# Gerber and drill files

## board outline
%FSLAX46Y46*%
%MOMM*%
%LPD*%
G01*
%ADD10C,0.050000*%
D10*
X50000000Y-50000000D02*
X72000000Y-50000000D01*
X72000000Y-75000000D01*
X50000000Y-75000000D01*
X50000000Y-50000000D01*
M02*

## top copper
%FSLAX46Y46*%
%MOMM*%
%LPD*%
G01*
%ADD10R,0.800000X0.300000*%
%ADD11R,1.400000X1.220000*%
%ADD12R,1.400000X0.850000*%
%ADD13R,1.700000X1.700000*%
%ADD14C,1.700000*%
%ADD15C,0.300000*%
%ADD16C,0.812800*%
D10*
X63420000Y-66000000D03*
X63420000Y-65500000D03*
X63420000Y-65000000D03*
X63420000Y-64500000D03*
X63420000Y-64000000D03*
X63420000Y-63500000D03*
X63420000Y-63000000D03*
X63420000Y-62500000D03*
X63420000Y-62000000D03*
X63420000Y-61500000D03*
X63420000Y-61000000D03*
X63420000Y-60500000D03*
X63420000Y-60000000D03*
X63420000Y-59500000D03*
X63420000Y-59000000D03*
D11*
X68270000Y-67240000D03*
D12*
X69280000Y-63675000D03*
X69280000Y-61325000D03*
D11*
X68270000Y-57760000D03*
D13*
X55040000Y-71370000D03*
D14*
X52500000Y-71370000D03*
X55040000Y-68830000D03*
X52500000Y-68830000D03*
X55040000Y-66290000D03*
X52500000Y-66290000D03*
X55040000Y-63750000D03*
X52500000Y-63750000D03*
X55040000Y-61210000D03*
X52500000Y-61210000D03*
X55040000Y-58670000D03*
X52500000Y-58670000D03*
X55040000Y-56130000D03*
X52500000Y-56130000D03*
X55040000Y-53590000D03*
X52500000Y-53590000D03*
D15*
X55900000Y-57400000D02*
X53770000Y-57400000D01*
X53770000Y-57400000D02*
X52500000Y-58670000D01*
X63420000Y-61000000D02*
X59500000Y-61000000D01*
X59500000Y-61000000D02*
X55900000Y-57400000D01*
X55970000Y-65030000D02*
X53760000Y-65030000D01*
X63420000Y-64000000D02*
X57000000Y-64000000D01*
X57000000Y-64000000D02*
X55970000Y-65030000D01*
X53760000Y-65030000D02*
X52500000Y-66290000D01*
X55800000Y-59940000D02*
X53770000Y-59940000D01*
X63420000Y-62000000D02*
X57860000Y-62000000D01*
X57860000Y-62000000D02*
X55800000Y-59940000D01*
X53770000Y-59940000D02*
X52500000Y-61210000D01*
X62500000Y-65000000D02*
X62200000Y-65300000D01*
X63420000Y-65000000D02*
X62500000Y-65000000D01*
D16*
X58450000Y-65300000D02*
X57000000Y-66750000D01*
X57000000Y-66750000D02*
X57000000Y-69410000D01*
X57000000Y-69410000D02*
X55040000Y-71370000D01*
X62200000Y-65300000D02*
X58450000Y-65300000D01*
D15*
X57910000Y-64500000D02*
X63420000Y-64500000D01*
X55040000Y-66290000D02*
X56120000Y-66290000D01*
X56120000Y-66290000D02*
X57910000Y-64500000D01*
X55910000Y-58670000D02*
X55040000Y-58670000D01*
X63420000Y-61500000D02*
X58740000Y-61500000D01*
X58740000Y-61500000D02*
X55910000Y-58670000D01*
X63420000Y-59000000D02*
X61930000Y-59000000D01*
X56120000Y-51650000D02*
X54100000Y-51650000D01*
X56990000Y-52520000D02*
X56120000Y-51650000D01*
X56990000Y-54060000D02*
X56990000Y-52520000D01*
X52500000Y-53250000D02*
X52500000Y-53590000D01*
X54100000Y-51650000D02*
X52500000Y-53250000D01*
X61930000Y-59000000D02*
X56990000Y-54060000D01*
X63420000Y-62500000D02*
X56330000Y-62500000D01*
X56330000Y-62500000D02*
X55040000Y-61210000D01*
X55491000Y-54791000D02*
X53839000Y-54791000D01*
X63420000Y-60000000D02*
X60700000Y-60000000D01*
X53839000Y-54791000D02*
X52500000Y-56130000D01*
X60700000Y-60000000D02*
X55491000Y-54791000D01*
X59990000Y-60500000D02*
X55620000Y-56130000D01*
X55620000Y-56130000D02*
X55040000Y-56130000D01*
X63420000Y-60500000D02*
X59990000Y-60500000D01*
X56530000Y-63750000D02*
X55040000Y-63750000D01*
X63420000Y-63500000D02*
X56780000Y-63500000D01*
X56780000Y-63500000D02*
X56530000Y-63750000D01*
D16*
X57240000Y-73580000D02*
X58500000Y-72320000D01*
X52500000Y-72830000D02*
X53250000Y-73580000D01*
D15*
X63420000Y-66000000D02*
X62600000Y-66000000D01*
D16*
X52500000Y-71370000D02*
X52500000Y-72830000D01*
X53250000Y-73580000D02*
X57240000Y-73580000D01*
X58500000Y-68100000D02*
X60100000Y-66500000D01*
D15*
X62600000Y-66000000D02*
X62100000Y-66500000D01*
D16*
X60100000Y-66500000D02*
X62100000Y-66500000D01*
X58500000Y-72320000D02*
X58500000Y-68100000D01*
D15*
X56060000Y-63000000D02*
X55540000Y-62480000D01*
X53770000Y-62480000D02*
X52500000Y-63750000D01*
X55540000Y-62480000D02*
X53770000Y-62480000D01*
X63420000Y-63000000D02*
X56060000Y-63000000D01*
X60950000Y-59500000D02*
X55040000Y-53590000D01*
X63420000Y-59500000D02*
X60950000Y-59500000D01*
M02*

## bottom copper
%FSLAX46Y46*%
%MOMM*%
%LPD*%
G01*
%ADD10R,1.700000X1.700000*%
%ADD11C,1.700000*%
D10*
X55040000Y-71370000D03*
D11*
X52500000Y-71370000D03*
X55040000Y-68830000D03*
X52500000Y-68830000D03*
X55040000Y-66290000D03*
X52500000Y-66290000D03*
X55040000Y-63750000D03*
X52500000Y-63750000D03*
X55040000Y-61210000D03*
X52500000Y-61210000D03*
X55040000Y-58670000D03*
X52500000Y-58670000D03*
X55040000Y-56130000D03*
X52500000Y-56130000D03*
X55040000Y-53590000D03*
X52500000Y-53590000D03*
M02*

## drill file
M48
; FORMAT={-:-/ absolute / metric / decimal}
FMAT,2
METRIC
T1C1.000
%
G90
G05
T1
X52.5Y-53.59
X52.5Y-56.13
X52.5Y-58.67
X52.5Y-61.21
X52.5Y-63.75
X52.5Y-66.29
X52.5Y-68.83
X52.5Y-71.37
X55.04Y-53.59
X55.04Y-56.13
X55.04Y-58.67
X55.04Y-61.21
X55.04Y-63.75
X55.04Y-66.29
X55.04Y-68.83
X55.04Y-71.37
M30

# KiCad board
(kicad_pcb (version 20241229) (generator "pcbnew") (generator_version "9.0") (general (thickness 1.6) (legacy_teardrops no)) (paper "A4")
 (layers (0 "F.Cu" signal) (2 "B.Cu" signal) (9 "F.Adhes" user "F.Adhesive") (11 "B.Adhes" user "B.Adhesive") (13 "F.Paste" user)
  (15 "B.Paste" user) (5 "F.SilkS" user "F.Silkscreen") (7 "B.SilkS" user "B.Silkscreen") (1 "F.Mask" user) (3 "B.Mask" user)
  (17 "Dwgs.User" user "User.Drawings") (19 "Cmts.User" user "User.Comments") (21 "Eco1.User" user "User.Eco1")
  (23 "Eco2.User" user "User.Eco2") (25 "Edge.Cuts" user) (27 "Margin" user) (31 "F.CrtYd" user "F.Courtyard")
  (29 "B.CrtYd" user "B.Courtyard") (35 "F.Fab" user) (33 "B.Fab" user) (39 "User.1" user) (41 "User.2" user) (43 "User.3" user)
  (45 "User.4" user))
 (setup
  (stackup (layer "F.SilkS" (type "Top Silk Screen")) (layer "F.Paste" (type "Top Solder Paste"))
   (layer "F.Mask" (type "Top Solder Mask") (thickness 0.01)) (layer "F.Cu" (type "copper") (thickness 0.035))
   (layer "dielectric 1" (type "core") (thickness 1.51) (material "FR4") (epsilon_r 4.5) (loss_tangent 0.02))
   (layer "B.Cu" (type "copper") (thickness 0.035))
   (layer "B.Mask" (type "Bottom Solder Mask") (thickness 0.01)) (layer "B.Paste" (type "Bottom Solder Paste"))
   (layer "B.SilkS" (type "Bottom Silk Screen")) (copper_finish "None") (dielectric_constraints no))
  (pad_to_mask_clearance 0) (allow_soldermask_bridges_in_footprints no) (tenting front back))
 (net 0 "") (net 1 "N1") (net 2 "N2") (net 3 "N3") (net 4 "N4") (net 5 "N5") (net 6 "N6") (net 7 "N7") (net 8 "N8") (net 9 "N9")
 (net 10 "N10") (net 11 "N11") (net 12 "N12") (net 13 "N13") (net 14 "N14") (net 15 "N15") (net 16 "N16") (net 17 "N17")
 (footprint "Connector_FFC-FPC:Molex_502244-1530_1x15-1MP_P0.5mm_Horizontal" (layer "F.Cu") (at 66.5 62.5 90)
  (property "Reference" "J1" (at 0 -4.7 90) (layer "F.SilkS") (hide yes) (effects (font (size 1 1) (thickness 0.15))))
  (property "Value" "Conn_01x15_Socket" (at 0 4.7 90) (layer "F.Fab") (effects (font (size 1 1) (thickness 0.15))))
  (pad "1" smd rect (at -3.5 -3.08 90) (size 0.3 0.8) (layers "F.Cu" "F.Mask" "F.Paste") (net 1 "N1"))
  (pad "2" smd rect (at -3 -3.08 90) (size 0.3 0.8) (layers "F.Cu" "F.Mask" "F.Paste") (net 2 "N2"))
  (pad "3" smd rect (at -2.5 -3.08 90) (size 0.3 0.8) (layers "F.Cu" "F.Mask" "F.Paste") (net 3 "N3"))
  (pad "4" smd rect (at -2 -3.08 90) (size 0.3 0.8) (layers "F.Cu" "F.Mask" "F.Paste") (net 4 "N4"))
  (pad "5" smd rect (at -1.5 -3.08 90) (size 0.3 0.8) (layers "F.Cu" "F.Mask" "F.Paste") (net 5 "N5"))
  (pad "6" smd rect (at -1 -3.08 90) (size 0.3 0.8) (layers "F.Cu" "F.Mask" "F.Paste") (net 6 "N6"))
  (pad "7" smd rect (at -0.5 -3.08 90) (size 0.3 0.8) (layers "F.Cu" "F.Mask" "F.Paste") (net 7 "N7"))
  (pad "8" smd rect (at 0 -3.08 90) (size 0.3 0.8) (layers "F.Cu" "F.Mask" "F.Paste") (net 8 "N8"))
  (pad "9" smd rect (at 0.5 -3.08 90) (size 0.3 0.8) (layers "F.Cu" "F.Mask" "F.Paste") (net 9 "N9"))
  (pad "10" smd rect (at 1 -3.08 90) (size 0.3 0.8) (layers "F.Cu" "F.Mask" "F.Paste") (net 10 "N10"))
  (pad "11" smd rect (at 1.5 -3.08 90) (size 0.3 0.8) (layers "F.Cu" "F.Mask" "F.Paste") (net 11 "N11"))
  (pad "12" smd rect (at 2 -3.08 90) (size 0.3 0.8) (layers "F.Cu" "F.Mask" "F.Paste") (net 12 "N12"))
  (pad "13" smd rect (at 2.5 -3.08 90) (size 0.3 0.8) (layers "F.Cu" "F.Mask" "F.Paste") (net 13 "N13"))
  (pad "14" smd rect (at 3 -3.08 90) (size 0.3 0.8) (layers "F.Cu" "F.Mask" "F.Paste") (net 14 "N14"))
  (pad "15" smd rect (at 3.5 -3.08 90) (size 0.3 0.8) (layers "F.Cu" "F.Mask" "F.Paste") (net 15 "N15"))
  (pad "MP" smd rect (at -4.74 1.77 90) (size 1.22 1.4) (layers "F.Cu" "F.Mask" "F.Paste"))
  (pad "MP" smd rect (at -1.175 2.78 90) (size 0.85 1.4) (layers "F.Cu" "F.Mask" "F.Paste"))
  (pad "MP" smd rect (at 1.175 2.78 90) (size 0.85 1.4) (layers "F.Cu" "F.Mask" "F.Paste"))
  (pad "MP" smd rect (at 4.74 1.77 90) (size 1.22 1.4) (layers "F.Cu" "F.Mask" "F.Paste"))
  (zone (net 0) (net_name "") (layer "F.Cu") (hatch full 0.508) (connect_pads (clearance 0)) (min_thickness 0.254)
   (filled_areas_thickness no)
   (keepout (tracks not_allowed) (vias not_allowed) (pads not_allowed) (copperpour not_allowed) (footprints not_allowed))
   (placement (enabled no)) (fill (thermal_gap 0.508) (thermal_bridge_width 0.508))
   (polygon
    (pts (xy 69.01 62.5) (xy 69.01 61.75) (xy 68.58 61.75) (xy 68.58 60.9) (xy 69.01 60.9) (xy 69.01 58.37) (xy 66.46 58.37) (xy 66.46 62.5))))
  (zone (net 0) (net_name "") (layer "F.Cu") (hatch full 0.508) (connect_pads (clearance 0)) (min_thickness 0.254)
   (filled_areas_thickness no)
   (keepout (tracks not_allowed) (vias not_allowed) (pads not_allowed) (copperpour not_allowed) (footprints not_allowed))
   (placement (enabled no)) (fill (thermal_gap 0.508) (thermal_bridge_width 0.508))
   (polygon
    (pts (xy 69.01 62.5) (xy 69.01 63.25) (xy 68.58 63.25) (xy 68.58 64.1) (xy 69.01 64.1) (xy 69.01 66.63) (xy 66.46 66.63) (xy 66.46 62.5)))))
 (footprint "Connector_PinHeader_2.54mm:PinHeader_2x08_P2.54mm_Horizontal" (layer "F.Cu") (at 55.04 71.37 180)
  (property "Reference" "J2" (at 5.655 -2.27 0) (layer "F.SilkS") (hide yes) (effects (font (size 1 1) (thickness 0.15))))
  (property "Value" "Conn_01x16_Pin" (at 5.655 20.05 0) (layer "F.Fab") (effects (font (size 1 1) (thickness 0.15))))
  (pad "1" thru_hole rect (at 0 0 180) (size 1.7 1.7) (drill 1) (layers "*.Cu" "*.Mask") (remove_unused_layers no) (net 3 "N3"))
  (pad "2" thru_hole circle (at 2.54 0 180) (size 1.7 1.7) (drill 1) (layers "*.Cu" "*.Mask") (remove_unused_layers no) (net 1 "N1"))
  (pad "3" thru_hole circle (at 0 2.54 180) (size 1.7 1.7) (drill 1) (layers "*.Cu" "*.Mask") (remove_unused_layers no) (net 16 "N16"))
  (pad "4" thru_hole circle (at 2.54 2.54 180) (size 1.7 1.7) (drill 1) (layers "*.Cu" "*.Mask") (remove_unused_layers no) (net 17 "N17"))
  (pad "5" thru_hole circle (at 0 5.08 180) (size 1.7 1.7) (drill 1) (layers "*.Cu" "*.Mask") (remove_unused_layers no) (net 4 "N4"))
  (pad "6" thru_hole circle (at 2.54 5.08 180) (size 1.7 1.7) (drill 1) (layers "*.Cu" "*.Mask") (remove_unused_layers no) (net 5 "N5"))
  (pad "7" thru_hole circle (at 0 7.62 180) (size 1.7 1.7) (drill 1) (layers "*.Cu" "*.Mask") (remove_unused_layers no) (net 6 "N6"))
  (pad "8" thru_hole circle (at 2.54 7.62 180) (size 1.7 1.7) (drill 1) (layers "*.Cu" "*.Mask") (remove_unused_layers no) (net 7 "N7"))
  (pad "9" thru_hole circle (at 0 10.16 180) (size 1.7 1.7) (drill 1) (layers "*.Cu" "*.Mask") (remove_unused_layers no) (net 8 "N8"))
  (pad "10" thru_hole circle (at 2.54 10.16 180) (size 1.7 1.7) (drill 1) (layers "*.Cu" "*.Mask") (remove_unused_layers no) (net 9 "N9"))
  (pad "11" thru_hole circle (at 0 12.7 180) (size 1.7 1.7) (drill 1) (layers "*.Cu" "*.Mask") (remove_unused_layers no) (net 10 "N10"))
  (pad "12" thru_hole circle (at 2.54 12.7 180) (size 1.7 1.7) (drill 1) (layers "*.Cu" "*.Mask") (remove_unused_layers no) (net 11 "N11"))
  (pad "13" thru_hole circle (at 0 15.24 180) (size 1.7 1.7) (drill 1) (layers "*.Cu" "*.Mask") (remove_unused_layers no) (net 12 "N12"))
  (pad "14" thru_hole circle (at 2.54 15.24 180) (size 1.7 1.7) (drill 1) (layers "*.Cu" "*.Mask") (remove_unused_layers no) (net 13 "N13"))
  (pad "15" thru_hole circle (at 0 17.78 180) (size 1.7 1.7) (drill 1) (layers "*.Cu" "*.Mask") (remove_unused_layers no) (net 14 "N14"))
  (pad "16" thru_hole circle (at 2.54 17.78 180) (size 1.7 1.7) (drill 1) (layers "*.Cu" "*.Mask") (remove_unused_layers no) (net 15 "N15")))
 (gr_rect (start 50 50) (end 72 75) (stroke (width 0.05) (type solid)) (fill no) (layer "Edge.Cuts"))
 (segment (start 55.9 57.4) (end 53.77 57.4) (width 0.3) (layer "F.Cu") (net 11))
 (segment (start 53.77 57.4) (end 52.5 58.67) (width 0.3) (layer "F.Cu") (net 11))
 (segment (start 63.42 61) (end 59.5 61) (width 0.3) (layer "F.Cu") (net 11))
 (segment (start 59.5 61) (end 55.9 57.4) (width 0.3) (layer "F.Cu") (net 11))
 (segment (start 55.97 65.03) (end 53.76 65.03) (width 0.3) (layer "F.Cu") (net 5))
 (segment (start 63.42 64) (end 57 64) (width 0.3) (layer "F.Cu") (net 5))
 (segment (start 57 64) (end 55.97 65.03) (width 0.3) (layer "F.Cu") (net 5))
 (segment (start 53.76 65.03) (end 52.5 66.29) (width 0.3) (layer "F.Cu") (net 5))
 (segment (start 55.8 59.94) (end 53.77 59.94) (width 0.3) (layer "F.Cu") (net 9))
 (segment (start 63.42 62) (end 57.86 62) (width 0.3) (layer "F.Cu") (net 9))
 (segment (start 57.86 62) (end 55.8 59.94) (width 0.3) (layer "F.Cu") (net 9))
 (segment (start 53.77 59.94) (end 52.5 61.21) (width 0.3) (layer "F.Cu") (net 9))
 (segment (start 62.5 65) (end 62.2 65.3) (width 0.3) (layer "F.Cu") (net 3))
 (segment (start 63.42 65) (end 62.5 65) (width 0.3) (layer "F.Cu") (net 3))
 (segment (start 58.45 65.3) (end 57 66.75) (width 0.8128) (layer "F.Cu") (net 3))
 (segment (start 57 66.75) (end 57 69.41) (width 0.8128) (layer "F.Cu") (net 3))
 (segment (start 57 69.41) (end 55.04 71.37) (width 0.8128) (layer "F.Cu") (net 3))
 (segment (start 62.2 65.3) (end 58.45 65.3) (width 0.8128) (layer "F.Cu") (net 3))
 (segment (start 57.91 64.5) (end 63.42 64.5) (width 0.3) (layer "F.Cu") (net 4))
 (segment (start 55.04 66.29) (end 56.12 66.29) (width 0.3) (layer "F.Cu") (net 4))
 (segment (start 56.12 66.29) (end 57.91 64.5) (width 0.3) (layer "F.Cu") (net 4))
 (segment (start 55.91 58.67) (end 55.04 58.67) (width 0.3) (layer "F.Cu") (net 10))
 (segment (start 63.42 61.5) (end 58.74 61.5) (width 0.3) (layer "F.Cu") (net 10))
 (segment (start 58.74 61.5) (end 55.91 58.67) (width 0.3) (layer "F.Cu") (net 10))
 (segment (start 63.42 59) (end 61.93 59) (width 0.3) (layer "F.Cu") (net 15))
 (segment (start 56.12 51.65) (end 54.1 51.65) (width 0.3) (layer "F.Cu") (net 15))
 (segment (start 56.99 52.52) (end 56.12 51.65) (width 0.3) (layer "F.Cu") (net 15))
 (segment (start 56.99 54.06) (end 56.99 52.52) (width 0.3) (layer "F.Cu") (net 15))
 (segment (start 52.5 53.25) (end 52.5 53.59) (width 0.3) (layer "F.Cu") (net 15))
 (segment (start 54.1 51.65) (end 52.5 53.25) (width 0.3) (layer "F.Cu") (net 15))
 (segment (start 61.93 59) (end 56.99 54.06) (width 0.3) (layer "F.Cu") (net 15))
 (segment (start 63.42 62.5) (end 56.33 62.5) (width 0.3) (layer "F.Cu") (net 8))
 (segment (start 56.33 62.5) (end 55.04 61.21) (width 0.3) (layer "F.Cu") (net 8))
 (segment (start 55.491 54.791) (end 53.839 54.791) (width 0.3) (layer "F.Cu") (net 13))
 (segment (start 63.42 60) (end 60.7 60) (width 0.3) (layer "F.Cu") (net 13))
 (segment (start 53.839 54.791) (end 52.5 56.13) (width 0.3) (layer "F.Cu") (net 13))
 (segment (start 60.7 60) (end 55.491 54.791) (width 0.3) (layer "F.Cu") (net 13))
 (segment (start 59.99 60.5) (end 55.62 56.13) (width 0.3) (layer "F.Cu") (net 12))
 (segment (start 55.62 56.13) (end 55.04 56.13) (width 0.3) (layer "F.Cu") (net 12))
 (segment (start 63.42 60.5) (end 59.99 60.5) (width 0.3) (layer "F.Cu") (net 12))
 (segment (start 56.53 63.75) (end 55.04 63.75) (width 0.3) (layer "F.Cu") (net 6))
 (segment (start 63.42 63.5) (end 56.78 63.5) (width 0.3) (layer "F.Cu") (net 6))
 (segment (start 56.78 63.5) (end 56.53 63.75) (width 0.3) (layer "F.Cu") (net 6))
 (segment (start 57.24 73.58) (end 58.5 72.32) (width 0.8128) (layer "F.Cu") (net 1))
 (segment (start 52.5 72.83) (end 53.25 73.58) (width 0.8128) (layer "F.Cu") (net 1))
 (segment (start 63.42 66) (end 62.6 66) (width 0.3) (layer "F.Cu") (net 1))
 (segment (start 52.5 71.37) (end 52.5 72.83) (width 0.8128) (layer "F.Cu") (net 1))
 (segment (start 53.25 73.58) (end 57.24 73.58) (width 0.8128) (layer "F.Cu") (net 1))
 (segment (start 58.5 68.1) (end 60.1 66.5) (width 0.8128) (layer "F.Cu") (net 1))
 (segment (start 62.6 66) (end 62.1 66.5) (width 0.3) (layer "F.Cu") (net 1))
 (segment (start 60.1 66.5) (end 62.1 66.5) (width 0.8128) (layer "F.Cu") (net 1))
 (segment (start 58.5 72.32) (end 58.5 68.1) (width 0.8128) (layer "F.Cu") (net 1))
 (segment (start 56.06 63) (end 55.54 62.48) (width 0.3) (layer "F.Cu") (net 7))
 (segment (start 53.77 62.48) (end 52.5 63.75) (width 0.3) (layer "F.Cu") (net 7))
 (segment (start 55.54 62.48) (end 53.77 62.48) (width 0.3) (layer "F.Cu") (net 7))
 (segment (start 63.42 63) (end 56.06 63) (width 0.3) (layer "F.Cu") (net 7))
 (segment (start 60.95 59.5) (end 55.04 53.59) (width 0.3) (layer "F.Cu") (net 14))
 (segment (start 63.42 59.5) (end 60.95 59.5) (width 0.3) (layer "F.Cu") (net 14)))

